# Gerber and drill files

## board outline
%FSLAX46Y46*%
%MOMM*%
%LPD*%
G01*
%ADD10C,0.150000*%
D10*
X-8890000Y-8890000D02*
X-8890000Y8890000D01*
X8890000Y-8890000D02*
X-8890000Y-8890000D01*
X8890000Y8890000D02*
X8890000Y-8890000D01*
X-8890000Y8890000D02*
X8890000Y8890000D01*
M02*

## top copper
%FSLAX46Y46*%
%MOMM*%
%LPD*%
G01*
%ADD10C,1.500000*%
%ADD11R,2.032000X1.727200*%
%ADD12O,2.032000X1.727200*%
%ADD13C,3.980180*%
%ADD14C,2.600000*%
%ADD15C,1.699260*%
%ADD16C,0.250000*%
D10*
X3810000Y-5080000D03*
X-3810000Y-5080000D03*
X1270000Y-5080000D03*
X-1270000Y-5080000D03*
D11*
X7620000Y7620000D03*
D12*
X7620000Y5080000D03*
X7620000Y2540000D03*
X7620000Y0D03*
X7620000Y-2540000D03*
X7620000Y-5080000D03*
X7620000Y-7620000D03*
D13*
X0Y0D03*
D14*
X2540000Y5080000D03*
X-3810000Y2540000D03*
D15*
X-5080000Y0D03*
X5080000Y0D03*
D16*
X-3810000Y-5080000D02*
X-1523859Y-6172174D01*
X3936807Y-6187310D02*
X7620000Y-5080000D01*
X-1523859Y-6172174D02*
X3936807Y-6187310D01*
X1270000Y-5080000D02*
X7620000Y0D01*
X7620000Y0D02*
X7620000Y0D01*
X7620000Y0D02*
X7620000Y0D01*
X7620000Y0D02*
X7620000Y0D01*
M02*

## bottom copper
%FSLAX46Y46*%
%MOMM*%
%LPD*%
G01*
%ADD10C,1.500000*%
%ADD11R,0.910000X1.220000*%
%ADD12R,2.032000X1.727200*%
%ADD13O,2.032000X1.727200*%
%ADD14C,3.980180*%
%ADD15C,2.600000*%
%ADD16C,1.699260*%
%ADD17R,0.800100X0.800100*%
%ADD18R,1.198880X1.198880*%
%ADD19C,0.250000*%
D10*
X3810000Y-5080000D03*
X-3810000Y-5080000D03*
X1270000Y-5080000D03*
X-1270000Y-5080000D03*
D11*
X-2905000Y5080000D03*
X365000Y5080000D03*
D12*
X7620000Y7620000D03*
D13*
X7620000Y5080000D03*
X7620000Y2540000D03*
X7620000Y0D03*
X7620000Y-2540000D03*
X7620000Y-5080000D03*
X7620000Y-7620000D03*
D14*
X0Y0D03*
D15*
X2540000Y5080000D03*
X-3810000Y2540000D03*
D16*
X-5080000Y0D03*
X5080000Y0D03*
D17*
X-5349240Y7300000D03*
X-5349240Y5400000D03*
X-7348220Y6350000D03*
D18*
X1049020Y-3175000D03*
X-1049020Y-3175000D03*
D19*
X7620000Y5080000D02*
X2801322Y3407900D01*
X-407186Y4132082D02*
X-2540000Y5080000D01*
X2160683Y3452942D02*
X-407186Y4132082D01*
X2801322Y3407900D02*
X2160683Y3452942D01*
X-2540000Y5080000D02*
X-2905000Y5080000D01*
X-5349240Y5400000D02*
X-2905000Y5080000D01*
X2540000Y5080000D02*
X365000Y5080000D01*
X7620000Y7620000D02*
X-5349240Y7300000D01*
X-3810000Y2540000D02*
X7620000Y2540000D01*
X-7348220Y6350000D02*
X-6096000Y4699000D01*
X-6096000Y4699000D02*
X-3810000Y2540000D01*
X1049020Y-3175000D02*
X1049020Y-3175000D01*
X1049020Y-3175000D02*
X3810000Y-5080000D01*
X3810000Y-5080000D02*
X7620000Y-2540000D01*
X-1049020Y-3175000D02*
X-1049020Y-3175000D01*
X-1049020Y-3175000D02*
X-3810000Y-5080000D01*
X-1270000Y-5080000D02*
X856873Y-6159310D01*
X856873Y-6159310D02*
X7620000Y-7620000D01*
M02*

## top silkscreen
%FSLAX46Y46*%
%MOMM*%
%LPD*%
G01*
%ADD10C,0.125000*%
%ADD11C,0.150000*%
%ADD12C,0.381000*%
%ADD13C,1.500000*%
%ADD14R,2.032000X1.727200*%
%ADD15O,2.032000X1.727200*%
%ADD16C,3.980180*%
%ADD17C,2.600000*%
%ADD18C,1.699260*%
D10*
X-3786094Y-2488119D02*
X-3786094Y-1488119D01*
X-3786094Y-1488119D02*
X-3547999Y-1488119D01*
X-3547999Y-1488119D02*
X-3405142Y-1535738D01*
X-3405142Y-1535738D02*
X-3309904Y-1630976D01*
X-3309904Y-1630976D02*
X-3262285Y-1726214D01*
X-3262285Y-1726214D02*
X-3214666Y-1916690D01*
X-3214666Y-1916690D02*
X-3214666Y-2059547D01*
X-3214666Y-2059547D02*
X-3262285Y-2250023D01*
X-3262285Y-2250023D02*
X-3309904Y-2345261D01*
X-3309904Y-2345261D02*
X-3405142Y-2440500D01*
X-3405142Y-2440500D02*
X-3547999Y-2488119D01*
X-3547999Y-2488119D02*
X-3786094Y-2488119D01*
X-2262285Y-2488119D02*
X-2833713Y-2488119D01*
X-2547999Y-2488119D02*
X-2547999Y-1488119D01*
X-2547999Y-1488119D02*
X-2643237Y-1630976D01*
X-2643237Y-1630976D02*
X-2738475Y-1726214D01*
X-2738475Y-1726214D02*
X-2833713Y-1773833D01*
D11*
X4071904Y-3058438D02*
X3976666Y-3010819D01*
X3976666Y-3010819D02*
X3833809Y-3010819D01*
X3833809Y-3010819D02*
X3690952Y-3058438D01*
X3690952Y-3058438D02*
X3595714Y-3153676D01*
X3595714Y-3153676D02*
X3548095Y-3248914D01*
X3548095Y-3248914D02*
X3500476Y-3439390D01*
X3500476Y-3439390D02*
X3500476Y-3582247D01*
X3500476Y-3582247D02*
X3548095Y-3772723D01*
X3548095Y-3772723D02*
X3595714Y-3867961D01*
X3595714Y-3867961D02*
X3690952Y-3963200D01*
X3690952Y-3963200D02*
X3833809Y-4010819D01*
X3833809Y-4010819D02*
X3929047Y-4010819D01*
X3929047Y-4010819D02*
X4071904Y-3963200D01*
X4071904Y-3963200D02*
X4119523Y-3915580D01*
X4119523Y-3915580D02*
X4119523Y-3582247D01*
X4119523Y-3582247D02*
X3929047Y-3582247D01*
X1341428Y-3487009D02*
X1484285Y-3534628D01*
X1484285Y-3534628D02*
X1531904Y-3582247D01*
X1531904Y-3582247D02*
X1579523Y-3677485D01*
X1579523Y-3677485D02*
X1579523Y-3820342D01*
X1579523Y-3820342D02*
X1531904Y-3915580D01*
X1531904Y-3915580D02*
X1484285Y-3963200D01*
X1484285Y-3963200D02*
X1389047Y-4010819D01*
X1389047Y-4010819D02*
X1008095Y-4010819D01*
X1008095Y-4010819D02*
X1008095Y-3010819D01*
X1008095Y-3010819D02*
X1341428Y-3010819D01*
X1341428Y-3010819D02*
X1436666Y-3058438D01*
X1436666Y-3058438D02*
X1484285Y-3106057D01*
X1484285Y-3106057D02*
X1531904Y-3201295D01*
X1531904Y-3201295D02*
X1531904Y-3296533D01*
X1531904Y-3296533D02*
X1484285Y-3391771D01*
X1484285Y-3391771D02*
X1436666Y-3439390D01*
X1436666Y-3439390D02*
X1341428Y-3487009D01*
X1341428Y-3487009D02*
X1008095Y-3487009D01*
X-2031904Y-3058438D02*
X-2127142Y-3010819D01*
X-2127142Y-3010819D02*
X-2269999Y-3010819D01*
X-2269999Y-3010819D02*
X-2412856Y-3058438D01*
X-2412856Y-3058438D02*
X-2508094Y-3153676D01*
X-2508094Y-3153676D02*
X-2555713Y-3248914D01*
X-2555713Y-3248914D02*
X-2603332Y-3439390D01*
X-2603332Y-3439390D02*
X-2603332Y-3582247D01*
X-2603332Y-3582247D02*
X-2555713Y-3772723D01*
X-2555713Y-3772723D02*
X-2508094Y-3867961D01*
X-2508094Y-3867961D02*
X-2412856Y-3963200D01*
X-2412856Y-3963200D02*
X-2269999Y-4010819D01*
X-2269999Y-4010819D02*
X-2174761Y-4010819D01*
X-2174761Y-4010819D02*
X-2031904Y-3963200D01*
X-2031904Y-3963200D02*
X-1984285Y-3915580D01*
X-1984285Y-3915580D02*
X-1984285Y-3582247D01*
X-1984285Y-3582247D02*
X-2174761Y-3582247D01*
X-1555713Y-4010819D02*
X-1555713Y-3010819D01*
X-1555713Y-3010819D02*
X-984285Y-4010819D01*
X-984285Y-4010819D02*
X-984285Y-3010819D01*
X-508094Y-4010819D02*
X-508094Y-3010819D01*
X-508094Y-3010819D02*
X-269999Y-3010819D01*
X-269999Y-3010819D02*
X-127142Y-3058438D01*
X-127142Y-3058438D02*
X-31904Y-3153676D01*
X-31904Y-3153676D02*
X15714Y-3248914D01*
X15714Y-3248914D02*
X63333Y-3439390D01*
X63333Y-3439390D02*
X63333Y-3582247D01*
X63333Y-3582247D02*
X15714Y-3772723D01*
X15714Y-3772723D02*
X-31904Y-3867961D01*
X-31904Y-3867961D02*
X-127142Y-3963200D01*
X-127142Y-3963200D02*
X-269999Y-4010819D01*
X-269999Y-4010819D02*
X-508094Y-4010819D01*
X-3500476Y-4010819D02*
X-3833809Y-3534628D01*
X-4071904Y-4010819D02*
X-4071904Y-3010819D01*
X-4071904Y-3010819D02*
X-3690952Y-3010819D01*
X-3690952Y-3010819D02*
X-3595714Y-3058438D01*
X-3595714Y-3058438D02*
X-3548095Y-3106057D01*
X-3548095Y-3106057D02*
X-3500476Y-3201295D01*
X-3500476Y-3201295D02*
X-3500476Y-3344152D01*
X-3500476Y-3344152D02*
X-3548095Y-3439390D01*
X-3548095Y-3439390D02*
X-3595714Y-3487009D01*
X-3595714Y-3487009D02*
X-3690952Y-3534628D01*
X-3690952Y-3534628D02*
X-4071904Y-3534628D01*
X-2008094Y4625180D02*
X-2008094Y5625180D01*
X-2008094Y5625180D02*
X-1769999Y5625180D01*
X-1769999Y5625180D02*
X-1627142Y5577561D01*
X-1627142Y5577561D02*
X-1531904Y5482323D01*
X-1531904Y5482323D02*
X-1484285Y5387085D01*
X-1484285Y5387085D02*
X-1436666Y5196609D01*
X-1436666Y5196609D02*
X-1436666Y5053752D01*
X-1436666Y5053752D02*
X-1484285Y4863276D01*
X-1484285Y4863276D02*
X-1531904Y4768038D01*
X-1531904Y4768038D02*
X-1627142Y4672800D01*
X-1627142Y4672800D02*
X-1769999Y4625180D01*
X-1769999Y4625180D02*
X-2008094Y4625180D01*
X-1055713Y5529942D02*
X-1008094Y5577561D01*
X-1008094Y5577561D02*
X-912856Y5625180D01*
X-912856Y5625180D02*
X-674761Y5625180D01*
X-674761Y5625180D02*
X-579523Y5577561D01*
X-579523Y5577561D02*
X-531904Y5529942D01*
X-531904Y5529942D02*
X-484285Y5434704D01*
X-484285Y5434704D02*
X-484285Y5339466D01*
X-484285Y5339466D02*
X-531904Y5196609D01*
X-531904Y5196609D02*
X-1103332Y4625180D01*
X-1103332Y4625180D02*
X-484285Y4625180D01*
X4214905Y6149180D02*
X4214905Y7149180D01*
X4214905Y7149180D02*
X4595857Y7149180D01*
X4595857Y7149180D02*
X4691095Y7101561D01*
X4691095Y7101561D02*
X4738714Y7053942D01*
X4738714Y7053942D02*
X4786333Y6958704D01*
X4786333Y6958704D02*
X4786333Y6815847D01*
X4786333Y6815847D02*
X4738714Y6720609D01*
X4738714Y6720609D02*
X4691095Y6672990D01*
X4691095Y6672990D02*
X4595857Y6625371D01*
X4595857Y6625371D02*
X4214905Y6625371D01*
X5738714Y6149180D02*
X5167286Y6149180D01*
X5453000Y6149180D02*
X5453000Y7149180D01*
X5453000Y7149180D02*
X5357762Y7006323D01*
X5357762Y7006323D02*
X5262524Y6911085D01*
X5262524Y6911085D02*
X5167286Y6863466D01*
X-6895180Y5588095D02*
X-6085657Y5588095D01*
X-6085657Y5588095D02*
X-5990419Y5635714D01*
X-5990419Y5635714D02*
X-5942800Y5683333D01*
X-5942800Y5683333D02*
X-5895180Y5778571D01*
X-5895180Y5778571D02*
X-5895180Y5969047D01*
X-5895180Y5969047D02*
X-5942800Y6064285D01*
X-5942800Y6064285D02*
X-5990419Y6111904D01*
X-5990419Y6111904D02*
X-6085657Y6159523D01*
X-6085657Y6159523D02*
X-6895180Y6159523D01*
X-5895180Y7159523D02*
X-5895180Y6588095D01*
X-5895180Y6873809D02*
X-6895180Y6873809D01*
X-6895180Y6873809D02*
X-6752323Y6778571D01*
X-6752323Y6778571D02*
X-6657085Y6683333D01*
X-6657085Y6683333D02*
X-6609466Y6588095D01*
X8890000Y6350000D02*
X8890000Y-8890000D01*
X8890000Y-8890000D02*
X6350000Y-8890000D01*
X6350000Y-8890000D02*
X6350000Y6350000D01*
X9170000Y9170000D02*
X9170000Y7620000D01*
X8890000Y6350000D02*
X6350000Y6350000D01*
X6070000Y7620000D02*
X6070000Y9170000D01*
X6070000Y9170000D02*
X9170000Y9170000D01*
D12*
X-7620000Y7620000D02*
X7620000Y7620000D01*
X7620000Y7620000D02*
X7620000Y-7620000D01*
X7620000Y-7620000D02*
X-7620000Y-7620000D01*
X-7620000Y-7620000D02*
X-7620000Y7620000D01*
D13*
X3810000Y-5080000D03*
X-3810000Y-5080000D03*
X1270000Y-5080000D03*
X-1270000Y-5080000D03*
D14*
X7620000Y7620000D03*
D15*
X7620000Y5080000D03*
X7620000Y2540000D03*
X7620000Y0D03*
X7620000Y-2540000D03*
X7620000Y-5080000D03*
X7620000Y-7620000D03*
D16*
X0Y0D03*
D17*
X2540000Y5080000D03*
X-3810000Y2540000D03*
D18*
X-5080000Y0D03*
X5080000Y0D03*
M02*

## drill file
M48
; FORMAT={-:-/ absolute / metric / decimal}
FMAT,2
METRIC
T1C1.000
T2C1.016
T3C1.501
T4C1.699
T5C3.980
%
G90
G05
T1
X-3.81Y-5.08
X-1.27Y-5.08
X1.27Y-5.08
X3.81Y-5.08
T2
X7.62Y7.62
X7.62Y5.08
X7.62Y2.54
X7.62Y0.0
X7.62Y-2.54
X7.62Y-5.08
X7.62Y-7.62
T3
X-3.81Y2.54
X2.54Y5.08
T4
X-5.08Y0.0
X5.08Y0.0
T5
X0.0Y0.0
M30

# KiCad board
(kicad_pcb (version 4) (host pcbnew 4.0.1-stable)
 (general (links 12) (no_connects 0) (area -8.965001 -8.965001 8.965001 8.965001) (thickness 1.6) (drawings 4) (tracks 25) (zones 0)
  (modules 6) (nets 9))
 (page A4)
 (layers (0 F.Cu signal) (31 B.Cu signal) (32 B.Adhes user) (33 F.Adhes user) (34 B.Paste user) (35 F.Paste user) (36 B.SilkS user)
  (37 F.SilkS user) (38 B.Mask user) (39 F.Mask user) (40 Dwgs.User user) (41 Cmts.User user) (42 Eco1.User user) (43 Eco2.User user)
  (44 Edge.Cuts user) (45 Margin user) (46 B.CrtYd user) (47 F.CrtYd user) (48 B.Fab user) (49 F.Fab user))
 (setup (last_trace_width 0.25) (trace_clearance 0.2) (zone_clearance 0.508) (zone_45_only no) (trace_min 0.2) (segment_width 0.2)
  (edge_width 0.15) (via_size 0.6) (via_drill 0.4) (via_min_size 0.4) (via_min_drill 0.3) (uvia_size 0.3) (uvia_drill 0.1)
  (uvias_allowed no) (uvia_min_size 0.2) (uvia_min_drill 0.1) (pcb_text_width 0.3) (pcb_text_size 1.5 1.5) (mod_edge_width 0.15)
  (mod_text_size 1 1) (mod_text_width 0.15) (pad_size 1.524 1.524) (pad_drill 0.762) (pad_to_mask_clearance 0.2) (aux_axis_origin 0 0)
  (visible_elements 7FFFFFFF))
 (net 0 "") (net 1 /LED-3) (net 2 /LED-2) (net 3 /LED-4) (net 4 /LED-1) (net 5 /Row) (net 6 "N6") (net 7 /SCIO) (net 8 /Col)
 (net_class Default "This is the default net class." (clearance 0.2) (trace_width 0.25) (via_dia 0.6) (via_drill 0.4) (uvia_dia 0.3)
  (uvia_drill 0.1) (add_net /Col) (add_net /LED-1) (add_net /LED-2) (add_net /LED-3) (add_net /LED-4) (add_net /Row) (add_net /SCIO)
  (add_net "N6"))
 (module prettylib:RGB (layer F.Cu) (at 0 0)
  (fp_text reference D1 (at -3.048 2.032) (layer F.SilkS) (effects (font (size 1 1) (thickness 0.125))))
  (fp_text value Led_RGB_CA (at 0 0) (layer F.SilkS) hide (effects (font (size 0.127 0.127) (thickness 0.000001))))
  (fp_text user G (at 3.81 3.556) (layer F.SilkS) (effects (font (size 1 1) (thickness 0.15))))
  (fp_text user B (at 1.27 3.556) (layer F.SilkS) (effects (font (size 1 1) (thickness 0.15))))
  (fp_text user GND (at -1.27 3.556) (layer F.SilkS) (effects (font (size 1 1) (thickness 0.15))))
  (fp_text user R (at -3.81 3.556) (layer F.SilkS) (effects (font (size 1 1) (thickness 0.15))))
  (pad 3 thru_hole circle (at 3.81 5.08) (size 1.5 1.5) (drill 1) (layers *.Cu *.Mask F.SilkS) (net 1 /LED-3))
  (pad 2 thru_hole circle (at -3.81 5.08) (size 1.5 1.5) (drill 1) (layers *.Cu *.Mask F.SilkS) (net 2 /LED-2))
  (pad 4 thru_hole circle (at 1.27 5.08) (size 1.5 1.5) (drill 1) (layers *.Cu *.Mask F.SilkS) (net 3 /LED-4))
  (pad 1 thru_hole circle (at -1.27 5.08) (size 1.5 1.5) (drill 1) (layers *.Cu *.Mask F.SilkS) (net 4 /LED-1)))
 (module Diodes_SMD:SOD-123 (layer B.Cu) (at -1.27 -5.08)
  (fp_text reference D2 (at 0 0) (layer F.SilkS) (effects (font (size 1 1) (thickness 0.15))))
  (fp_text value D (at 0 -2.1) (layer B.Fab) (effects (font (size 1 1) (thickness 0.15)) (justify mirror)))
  (pad 1 smd rect (at -1.635 0) (size 0.91 1.22) (layers B.Cu B.Paste B.Mask) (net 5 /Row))
  (pad 2 smd rect (at 1.635 0) (size 0.91 1.22) (layers B.Cu B.Paste B.Mask) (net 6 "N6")))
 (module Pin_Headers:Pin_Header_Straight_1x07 (layer F.Cu) (at 7.62 -7.62)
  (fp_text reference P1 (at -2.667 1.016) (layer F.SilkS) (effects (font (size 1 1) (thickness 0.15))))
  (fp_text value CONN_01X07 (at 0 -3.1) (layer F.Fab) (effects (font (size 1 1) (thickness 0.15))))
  (fp_line (start 1.27 1.27) (end 1.27 16.51) (layer F.SilkS) (width 0.15))
  (fp_line (start 1.27 16.51) (end -1.27 16.51) (layer F.SilkS) (width 0.15))
  (fp_line (start -1.27 16.51) (end -1.27 1.27) (layer F.SilkS) (width 0.15))
  (fp_line (start 1.55 -1.55) (end 1.55 0) (layer F.SilkS) (width 0.15))
  (fp_line (start 1.27 1.27) (end -1.27 1.27) (layer F.SilkS) (width 0.15))
  (fp_line (start -1.55 0) (end -1.55 -1.55) (layer F.SilkS) (width 0.15))
  (fp_line (start -1.55 -1.55) (end 1.55 -1.55) (layer F.SilkS) (width 0.15))
  (pad 1 thru_hole rect (at 0 0) (size 2.032 1.7272) (drill 1.016) (layers *.Cu *.Mask F.SilkS) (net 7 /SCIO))
  (pad 2 thru_hole oval (at 0 2.54) (size 2.032 1.7272) (drill 1.016) (layers *.Cu *.Mask F.SilkS) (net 5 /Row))
  (pad 3 thru_hole oval (at 0 5.08) (size 2.032 1.7272) (drill 1.016) (layers *.Cu *.Mask F.SilkS) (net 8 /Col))
  (pad 4 thru_hole oval (at 0 7.62) (size 2.032 1.7272) (drill 1.016) (layers *.Cu *.Mask F.SilkS) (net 3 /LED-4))
  (pad 5 thru_hole oval (at 0 10.16) (size 2.032 1.7272) (drill 1.016) (layers *.Cu *.Mask F.SilkS) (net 1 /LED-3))
  (pad 6 thru_hole oval (at 0 12.7) (size 2.032 1.7272) (drill 1.016) (layers *.Cu *.Mask F.SilkS) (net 2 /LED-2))
  (pad 7 thru_hole oval (at 0 15.24) (size 2.032 1.7272) (drill 1.016) (layers *.Cu *.Mask F.SilkS) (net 4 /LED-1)))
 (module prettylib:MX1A (layer F.Cu) (at 0 0)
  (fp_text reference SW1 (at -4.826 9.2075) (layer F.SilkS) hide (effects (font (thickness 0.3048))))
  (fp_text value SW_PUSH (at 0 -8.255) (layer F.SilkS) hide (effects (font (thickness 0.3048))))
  (fp_line (start -7.62 -7.62) (end 7.62 -7.62) (layer F.SilkS) (width 0.381))
  (fp_line (start 7.62 -7.62) (end 7.62 7.62) (layer F.SilkS) (width 0.381))
  (fp_line (start 7.62 7.62) (end -7.62 7.62) (layer F.SilkS) (width 0.381))
  (fp_line (start -7.62 7.62) (end -7.62 -7.62) (layer F.SilkS) (width 0.381))
  (pad 0 thru_hole circle (at 0 0) (size 3.98018 3.98018) (drill 3.98018) (layers *.Cu *.Mask F.SilkS))
  (pad 2 thru_hole circle (at 2.54 -5.08) (size 2.6 2.6) (drill 1.5011) (layers *.Cu *.Mask F.SilkS) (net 6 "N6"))
  (pad 1 thru_hole circle (at -3.81 -2.54) (size 2.6 2.6) (drill 1.5011) (layers *.Cu *.Mask F.SilkS) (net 8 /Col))
  (pad "" thru_hole circle (at -5.08 0) (size 1.69926 1.69926) (drill 1.69926) (layers *.Cu *.Mask F.SilkS))
  (pad "" thru_hole circle (at 5.08 0) (size 1.69926 1.69926) (drill 1.69926) (layers *.Cu *.Mask F.SilkS)))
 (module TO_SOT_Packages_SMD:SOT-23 (layer B.Cu) (at -6.35 -6.35 270)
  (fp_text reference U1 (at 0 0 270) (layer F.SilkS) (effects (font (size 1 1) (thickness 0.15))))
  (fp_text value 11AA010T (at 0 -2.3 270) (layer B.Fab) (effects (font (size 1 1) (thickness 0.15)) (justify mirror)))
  (pad 1 smd rect (at -0.95 -1.00076 270) (size 0.8001 0.8001) (layers B.Cu B.Paste B.Mask) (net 7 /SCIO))
  (pad 2 smd rect (at 0.95 -1.00076 270) (size 0.8001 0.8001) (layers B.Cu B.Paste B.Mask) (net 5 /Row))
  (pad 3 smd rect (at 0 0.99822 270) (size 0.8001 0.8001) (layers B.Cu B.Paste B.Mask) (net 8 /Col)))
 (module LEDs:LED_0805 (layer B.Cu) (at 0 3.175)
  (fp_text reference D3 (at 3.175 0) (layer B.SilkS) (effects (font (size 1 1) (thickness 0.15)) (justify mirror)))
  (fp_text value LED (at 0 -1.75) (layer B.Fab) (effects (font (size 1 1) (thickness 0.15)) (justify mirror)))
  (pad 2 smd rect (at 1.04902 0 180) (size 1.19888 1.19888) (layers B.Cu B.Paste B.Mask) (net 1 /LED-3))
  (pad 1 smd rect (at -1.04902 0 180) (size 1.19888 1.19888) (layers B.Cu B.Paste B.Mask) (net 2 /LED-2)))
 (gr_line (start -8.89 8.89) (end -8.89 -8.89) (angle 90) (layer Edge.Cuts) (width 0.15))
 (gr_line (start 8.89 8.89) (end -8.89 8.89) (angle 90) (layer Edge.Cuts) (width 0.15))
 (gr_line (start 8.89 -8.89) (end 8.89 8.89) (angle 90) (layer Edge.Cuts) (width 0.15))
 (gr_line (start -8.89 -8.89) (end 8.89 -8.89) (angle 90) (layer Edge.Cuts) (width 0.15))
 (segment (start 7.62 -5.08) (end 2.801322 -3.4079) (width 0.25) (layer B.Cu) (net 5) (status 10))
 (segment (start -0.407186 -4.132082) (end -2.54 -5.08) (width 0.25) (layer B.Cu) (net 5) (status 20))
 (segment (start 2.160683 -3.452942) (end -0.407186 -4.132082) (width 0.25) (layer B.Cu) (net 5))
 (segment (start 2.801322 -3.4079) (end 2.160683 -3.452942) (width 0.25) (layer B.Cu) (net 5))
 (segment (start -2.54 -5.08) (end -2.905 -5.08) (width 0.25) (layer B.Cu) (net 5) (status 30))
 (segment (start -5.34924 -5.4) (end -2.905 -5.08) (width 0.25) (layer B.Cu) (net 5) (status 30))
 (segment (start 2.54 -5.08) (end 0.365 -5.08) (width 0.25) (layer B.Cu) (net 6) (status 30))
 (segment (start 7.62 -7.62) (end -5.34924 -7.3) (width 0.25) (layer B.Cu) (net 7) (status 30))
 (segment (start -3.81 -2.54) (end 7.62 -2.54) (width 0.25) (layer B.Cu) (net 8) (status 30))
 (segment (start -7.34822 -6.35) (end -6.096 -4.699) (width 0.25) (layer B.Cu) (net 8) (status 10))
 (segment (start -6.096 -4.699) (end -3.81 -2.54) (width 0.25) (layer B.Cu) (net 8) (status 20))
 (segment (start 1.04902 3.175) (end 1.04902 3.175) (width 0.25) (layer B.Cu) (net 1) (status C00000))
 (segment (start 1.04902 3.175) (end 3.81 5.08) (width 0.25) (layer B.Cu) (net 1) (status C00000))
 (segment (start 3.81 5.08) (end 7.62 2.54) (width 0.25) (layer B.Cu) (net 1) (status 30))
 (segment (start -1.04902 3.175) (end -1.04902 3.175) (width 0.25) (layer B.Cu) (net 2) (status C00000))
 (segment (start -1.04902 3.175) (end -3.81 5.08) (width 0.25) (layer B.Cu) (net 2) (status C00000))
 (segment (start -3.81 5.08) (end -1.523859 6.172174) (width 0.25) (layer F.Cu) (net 2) (status 10))
 (segment (start 3.936807 6.18731) (end 7.62 5.08) (width 0.25) (layer F.Cu) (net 2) (status 20))
 (segment (start -1.523859 6.172174) (end 3.936807 6.18731) (width 0.25) (layer F.Cu) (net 2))
 (segment (start 1.27 5.08) (end 7.62 0) (width 0.25) (layer F.Cu) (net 3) (status C00000))
 (segment (start 7.62 0) (end 7.62 0) (width 0.25) (layer F.Cu) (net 3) (status C00000))
 (segment (start 7.62 0) (end 7.62 0) (width 0.25) (layer F.Cu) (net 3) (status C00000))
 (segment (start 7.62 0) (end 7.62 0) (width 0.25) (layer F.Cu) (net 3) (status C00000))
 (segment (start -1.27 5.08) (end 0.856873 6.15931) (width 0.25) (layer B.Cu) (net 4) (status 10))
 (segment (start 0.856873 6.15931) (end 7.62 7.62) (width 0.25) (layer B.Cu) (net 4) (status 20)))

